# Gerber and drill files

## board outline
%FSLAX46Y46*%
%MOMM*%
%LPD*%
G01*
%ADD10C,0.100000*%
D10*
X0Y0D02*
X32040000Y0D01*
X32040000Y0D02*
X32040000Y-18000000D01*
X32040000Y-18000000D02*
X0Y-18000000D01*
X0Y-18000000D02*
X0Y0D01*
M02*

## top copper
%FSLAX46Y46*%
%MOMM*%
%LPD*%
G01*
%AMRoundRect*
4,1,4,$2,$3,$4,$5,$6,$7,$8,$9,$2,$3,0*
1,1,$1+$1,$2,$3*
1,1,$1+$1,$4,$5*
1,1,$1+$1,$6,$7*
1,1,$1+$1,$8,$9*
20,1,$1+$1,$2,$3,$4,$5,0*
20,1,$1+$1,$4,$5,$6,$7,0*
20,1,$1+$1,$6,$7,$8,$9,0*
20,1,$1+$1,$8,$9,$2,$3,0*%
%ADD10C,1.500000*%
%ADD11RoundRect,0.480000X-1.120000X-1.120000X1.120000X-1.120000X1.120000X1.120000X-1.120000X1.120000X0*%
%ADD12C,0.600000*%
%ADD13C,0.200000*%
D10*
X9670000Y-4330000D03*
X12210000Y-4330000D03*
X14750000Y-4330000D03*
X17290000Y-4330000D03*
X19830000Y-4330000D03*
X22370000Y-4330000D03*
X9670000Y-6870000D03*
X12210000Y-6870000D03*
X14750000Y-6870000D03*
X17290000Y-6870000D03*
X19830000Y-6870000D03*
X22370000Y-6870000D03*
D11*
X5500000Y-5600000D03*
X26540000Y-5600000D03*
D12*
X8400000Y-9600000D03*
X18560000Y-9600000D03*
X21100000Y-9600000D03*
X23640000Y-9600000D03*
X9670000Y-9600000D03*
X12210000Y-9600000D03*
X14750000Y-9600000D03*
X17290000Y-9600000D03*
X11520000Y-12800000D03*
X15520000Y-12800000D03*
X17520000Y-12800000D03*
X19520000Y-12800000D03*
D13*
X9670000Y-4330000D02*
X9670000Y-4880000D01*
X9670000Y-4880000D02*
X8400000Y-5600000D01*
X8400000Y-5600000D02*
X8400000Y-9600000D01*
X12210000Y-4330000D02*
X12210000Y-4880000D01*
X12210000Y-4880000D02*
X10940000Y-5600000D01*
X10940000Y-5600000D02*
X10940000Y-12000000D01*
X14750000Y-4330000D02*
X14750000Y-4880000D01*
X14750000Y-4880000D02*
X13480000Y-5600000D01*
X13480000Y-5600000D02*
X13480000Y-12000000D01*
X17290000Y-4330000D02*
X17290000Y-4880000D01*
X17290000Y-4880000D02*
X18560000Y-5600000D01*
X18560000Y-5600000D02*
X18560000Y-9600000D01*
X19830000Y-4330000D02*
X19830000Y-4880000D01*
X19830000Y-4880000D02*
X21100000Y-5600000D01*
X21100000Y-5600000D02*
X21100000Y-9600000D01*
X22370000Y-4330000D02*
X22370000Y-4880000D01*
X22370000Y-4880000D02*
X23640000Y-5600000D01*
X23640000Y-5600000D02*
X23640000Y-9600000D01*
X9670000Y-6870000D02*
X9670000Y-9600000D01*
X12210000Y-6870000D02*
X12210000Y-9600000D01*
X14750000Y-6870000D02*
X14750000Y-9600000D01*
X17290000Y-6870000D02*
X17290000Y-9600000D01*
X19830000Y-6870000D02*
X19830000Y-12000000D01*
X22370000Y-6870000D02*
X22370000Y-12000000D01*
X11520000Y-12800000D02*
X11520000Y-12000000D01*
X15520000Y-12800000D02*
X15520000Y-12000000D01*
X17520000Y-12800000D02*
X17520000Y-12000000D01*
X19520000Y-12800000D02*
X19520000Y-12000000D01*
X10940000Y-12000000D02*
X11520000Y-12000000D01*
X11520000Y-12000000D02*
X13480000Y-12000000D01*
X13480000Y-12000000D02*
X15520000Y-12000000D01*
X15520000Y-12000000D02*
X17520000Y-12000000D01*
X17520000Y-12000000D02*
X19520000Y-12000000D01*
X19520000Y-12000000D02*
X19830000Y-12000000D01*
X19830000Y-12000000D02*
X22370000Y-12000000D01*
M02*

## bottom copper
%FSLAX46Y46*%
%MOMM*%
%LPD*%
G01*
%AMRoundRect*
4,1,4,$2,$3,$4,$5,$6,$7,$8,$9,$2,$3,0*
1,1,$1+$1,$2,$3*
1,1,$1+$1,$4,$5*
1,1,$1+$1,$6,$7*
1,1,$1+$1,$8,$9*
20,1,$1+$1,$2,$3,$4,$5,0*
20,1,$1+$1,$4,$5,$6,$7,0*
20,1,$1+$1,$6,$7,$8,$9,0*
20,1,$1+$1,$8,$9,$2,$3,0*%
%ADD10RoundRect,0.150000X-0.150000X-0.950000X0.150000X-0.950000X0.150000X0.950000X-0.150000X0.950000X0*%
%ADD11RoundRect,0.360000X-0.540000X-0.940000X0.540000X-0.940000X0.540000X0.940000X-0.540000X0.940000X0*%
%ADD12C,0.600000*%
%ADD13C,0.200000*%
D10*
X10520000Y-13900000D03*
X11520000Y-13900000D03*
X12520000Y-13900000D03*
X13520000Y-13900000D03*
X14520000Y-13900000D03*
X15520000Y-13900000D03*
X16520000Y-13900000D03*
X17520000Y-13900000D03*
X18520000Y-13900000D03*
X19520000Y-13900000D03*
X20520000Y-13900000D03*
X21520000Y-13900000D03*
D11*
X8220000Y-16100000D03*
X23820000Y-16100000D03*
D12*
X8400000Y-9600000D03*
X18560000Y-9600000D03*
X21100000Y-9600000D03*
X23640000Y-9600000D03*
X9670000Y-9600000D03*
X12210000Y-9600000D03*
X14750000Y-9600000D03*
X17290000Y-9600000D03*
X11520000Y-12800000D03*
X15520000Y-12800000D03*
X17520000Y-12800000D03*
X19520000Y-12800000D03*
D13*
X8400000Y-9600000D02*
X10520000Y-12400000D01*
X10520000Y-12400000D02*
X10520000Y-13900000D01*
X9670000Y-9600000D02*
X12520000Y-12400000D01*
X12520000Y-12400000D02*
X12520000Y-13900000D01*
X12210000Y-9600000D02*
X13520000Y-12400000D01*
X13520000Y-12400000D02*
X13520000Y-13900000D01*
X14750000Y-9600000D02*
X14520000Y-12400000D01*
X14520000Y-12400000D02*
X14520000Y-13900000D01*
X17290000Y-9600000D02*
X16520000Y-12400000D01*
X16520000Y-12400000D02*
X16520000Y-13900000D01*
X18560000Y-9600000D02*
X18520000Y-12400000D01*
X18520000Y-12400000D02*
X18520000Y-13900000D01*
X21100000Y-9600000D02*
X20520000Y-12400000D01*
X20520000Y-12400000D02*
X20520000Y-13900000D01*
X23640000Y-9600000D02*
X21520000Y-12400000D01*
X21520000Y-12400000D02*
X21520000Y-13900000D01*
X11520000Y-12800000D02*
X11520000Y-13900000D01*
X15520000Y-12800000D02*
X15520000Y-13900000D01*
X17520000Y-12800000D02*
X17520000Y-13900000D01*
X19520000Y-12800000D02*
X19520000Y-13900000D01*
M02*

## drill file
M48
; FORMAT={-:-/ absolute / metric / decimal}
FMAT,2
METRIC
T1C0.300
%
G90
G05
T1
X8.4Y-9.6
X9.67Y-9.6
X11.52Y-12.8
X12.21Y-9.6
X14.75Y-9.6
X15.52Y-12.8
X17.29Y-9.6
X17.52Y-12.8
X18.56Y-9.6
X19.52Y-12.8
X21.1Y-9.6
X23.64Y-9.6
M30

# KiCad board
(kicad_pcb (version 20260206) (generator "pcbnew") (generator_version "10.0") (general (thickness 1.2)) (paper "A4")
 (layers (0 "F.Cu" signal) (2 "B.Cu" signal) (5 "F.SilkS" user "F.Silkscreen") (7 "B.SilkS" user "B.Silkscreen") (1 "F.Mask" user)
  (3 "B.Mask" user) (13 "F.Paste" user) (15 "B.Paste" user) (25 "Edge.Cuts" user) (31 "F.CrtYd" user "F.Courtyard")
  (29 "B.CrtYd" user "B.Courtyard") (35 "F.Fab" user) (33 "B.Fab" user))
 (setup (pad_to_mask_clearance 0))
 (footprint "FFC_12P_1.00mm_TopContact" (at 16.02 15) (layer "B.Cu")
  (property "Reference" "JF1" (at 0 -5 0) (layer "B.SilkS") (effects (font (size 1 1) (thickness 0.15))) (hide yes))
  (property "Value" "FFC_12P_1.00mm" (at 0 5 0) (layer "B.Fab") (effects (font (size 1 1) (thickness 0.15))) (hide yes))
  (pad "1" smd roundrect (at -5.500 -1.1) (size 0.6 2.2) (layers "B.Cu" "B.Mask" "B.Paste") (roundrect_rratio 0.25) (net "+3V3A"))
  (pad "2" smd roundrect (at -4.500 -1.1) (size 0.6 2.2) (layers "B.Cu" "B.Mask" "B.Paste") (roundrect_rratio 0.25) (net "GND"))
  (pad "3" smd roundrect (at -3.500 -1.1) (size 0.6 2.2) (layers "B.Cu" "B.Mask" "B.Paste") (roundrect_rratio 0.25) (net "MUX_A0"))
  (pad "4" smd roundrect (at -2.500 -1.1) (size 0.6 2.2) (layers "B.Cu" "B.Mask" "B.Paste") (roundrect_rratio 0.25) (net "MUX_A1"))
  (pad "5" smd roundrect (at -1.500 -1.1) (size 0.6 2.2) (layers "B.Cu" "B.Mask" "B.Paste") (roundrect_rratio 0.25) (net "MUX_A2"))
  (pad "6" smd roundrect (at -0.500 -1.1) (size 0.6 2.2) (layers "B.Cu" "B.Mask" "B.Paste") (roundrect_rratio 0.25) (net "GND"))
  (pad "7" smd roundrect (at 0.500 -1.1) (size 0.6 2.2) (layers "B.Cu" "B.Mask" "B.Paste") (roundrect_rratio 0.25) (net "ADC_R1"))
  (pad "8" smd roundrect (at 1.500 -1.1) (size 0.6 2.2) (layers "B.Cu" "B.Mask" "B.Paste") (roundrect_rratio 0.25) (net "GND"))
  (pad "9" smd roundrect (at 2.500 -1.1) (size 0.6 2.2) (layers "B.Cu" "B.Mask" "B.Paste") (roundrect_rratio 0.25) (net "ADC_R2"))
  (pad "10" smd roundrect (at 3.500 -1.1) (size 0.6 2.2) (layers "B.Cu" "B.Mask" "B.Paste") (roundrect_rratio 0.25) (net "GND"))
  (pad "11" smd roundrect (at 4.500 -1.1) (size 0.6 2.2) (layers "B.Cu" "B.Mask" "B.Paste") (roundrect_rratio 0.25) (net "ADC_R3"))
  (pad "12" smd roundrect (at 5.500 -1.1) (size 0.6 2.2) (layers "B.Cu" "B.Mask" "B.Paste") (roundrect_rratio 0.25) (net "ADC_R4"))
  (pad "MP" smd roundrect (at -7.800 1.1) (size 1.8 2.6) (layers "B.Cu" "B.Mask" "B.Paste") (roundrect_rratio 0.2))
  (pad "MP" smd roundrect (at 7.800 1.1) (size 1.8 2.6) (layers "B.Cu" "B.Mask" "B.Paste") (roundrect_rratio 0.2)))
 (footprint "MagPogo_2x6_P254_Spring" (at 16.02 5.6) (layer "F.Cu")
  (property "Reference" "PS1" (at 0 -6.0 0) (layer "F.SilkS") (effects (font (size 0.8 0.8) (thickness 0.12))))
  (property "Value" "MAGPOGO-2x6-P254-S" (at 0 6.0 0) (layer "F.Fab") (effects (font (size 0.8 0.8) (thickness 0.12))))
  (pad "1" smd circle (at -6.35 -1.27) (size 1.5 1.5) (layers "F.Cu" "F.Paste" "F.Mask") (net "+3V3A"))
  (pad "2" smd circle (at -3.81 -1.27) (size 1.5 1.5) (layers "F.Cu" "F.Paste" "F.Mask") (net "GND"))
  (pad "3" smd circle (at -1.27 -1.27) (size 1.5 1.5) (layers "F.Cu" "F.Paste" "F.Mask") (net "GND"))
  (pad "4" smd circle (at 1.27 -1.27) (size 1.5 1.5) (layers "F.Cu" "F.Paste" "F.Mask") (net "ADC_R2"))
  (pad "5" smd circle (at 3.81 -1.27) (size 1.5 1.5) (layers "F.Cu" "F.Paste" "F.Mask") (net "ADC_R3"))
  (pad "6" smd circle (at 6.35 -1.27) (size 1.5 1.5) (layers "F.Cu" "F.Paste" "F.Mask") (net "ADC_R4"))
  (pad "7" smd circle (at -6.35 1.27) (size 1.5 1.5) (layers "F.Cu" "F.Paste" "F.Mask") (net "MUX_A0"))
  (pad "8" smd circle (at -3.81 1.27) (size 1.5 1.5) (layers "F.Cu" "F.Paste" "F.Mask") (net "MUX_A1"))
  (pad "9" smd circle (at -1.27 1.27) (size 1.5 1.5) (layers "F.Cu" "F.Paste" "F.Mask") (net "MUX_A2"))
  (pad "10" smd circle (at 1.27 1.27) (size 1.5 1.5) (layers "F.Cu" "F.Paste" "F.Mask") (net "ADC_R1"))
  (pad "11" smd circle (at 3.81 1.27) (size 1.5 1.5) (layers "F.Cu" "F.Paste" "F.Mask") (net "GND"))
  (pad "12" smd circle (at 6.35 1.27) (size 1.5 1.5) (layers "F.Cu" "F.Paste" "F.Mask") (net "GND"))
  (pad "MP1" smd roundrect (at -10.52 0) (size 3.2 3.2) (roundrect_rratio 0.15) (layers "F.Cu" "F.Paste" "F.Mask"))
  (pad "MP2" smd roundrect (at 10.52 0) (size 3.2 3.2) (roundrect_rratio 0.15) (layers "F.Cu" "F.Paste" "F.Mask")))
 (gr_line (start 0 0) (end 32.04 0) (stroke (width 0.1) (type solid)) (layer "Edge.Cuts"))
 (gr_line (start 32.04 0) (end 32.04 18) (stroke (width 0.1) (type solid)) (layer "Edge.Cuts"))
 (gr_line (start 32.04 18) (end 0 18) (stroke (width 0.1) (type solid)) (layer "Edge.Cuts"))
 (gr_line (start 0 18) (end 0 0) (stroke (width 0.1) (type solid)) (layer "Edge.Cuts"))
 (segment (start 9.67 4.33) (end 9.67 4.88) (width 0.2) (layer "F.Cu") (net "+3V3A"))
 (segment (start 9.67 4.88) (end 8.4 5.6) (width 0.2) (layer "F.Cu") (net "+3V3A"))
 (segment (start 8.4 5.6) (end 8.4 9.6) (width 0.2) (layer "F.Cu") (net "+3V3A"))
 (via (at 8.4 9.6) (size 0.6) (drill 0.3) (layers "F.Cu" "B.Cu") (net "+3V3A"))
 (segment (start 12.21 4.33) (end 12.21 4.88) (width 0.2) (layer "F.Cu") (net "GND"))
 (segment (start 12.21 4.88) (end 10.94 5.6) (width 0.2) (layer "F.Cu") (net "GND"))
 (segment (start 10.94 5.6) (end 10.94 12) (width 0.2) (layer "F.Cu") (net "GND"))
 (segment (start 14.75 4.33) (end 14.75 4.88) (width 0.2) (layer "F.Cu") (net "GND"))
 (segment (start 14.75 4.88) (end 13.48 5.6) (width 0.2) (layer "F.Cu") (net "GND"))
 (segment (start 13.48 5.6) (end 13.48 12) (width 0.2) (layer "F.Cu") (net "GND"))
 (segment (start 17.29 4.33) (end 17.29 4.88) (width 0.2) (layer "F.Cu") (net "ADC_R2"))
 (segment (start 17.29 4.88) (end 18.56 5.6) (width 0.2) (layer "F.Cu") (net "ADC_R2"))
 (segment (start 18.56 5.6) (end 18.56 9.6) (width 0.2) (layer "F.Cu") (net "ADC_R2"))
 (via (at 18.56 9.6) (size 0.6) (drill 0.3) (layers "F.Cu" "B.Cu") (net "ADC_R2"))
 (segment (start 19.83 4.33) (end 19.83 4.88) (width 0.2) (layer "F.Cu") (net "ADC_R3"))
 (segment (start 19.83 4.88) (end 21.1 5.6) (width 0.2) (layer "F.Cu") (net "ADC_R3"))
 (segment (start 21.1 5.6) (end 21.1 9.6) (width 0.2) (layer "F.Cu") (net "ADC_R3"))
 (via (at 21.1 9.6) (size 0.6) (drill 0.3) (layers "F.Cu" "B.Cu") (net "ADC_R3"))
 (segment (start 22.37 4.33) (end 22.37 4.88) (width 0.2) (layer "F.Cu") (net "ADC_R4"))
 (segment (start 22.37 4.88) (end 23.64 5.6) (width 0.2) (layer "F.Cu") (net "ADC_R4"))
 (segment (start 23.64 5.6) (end 23.64 9.6) (width 0.2) (layer "F.Cu") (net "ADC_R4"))
 (via (at 23.64 9.6) (size 0.6) (drill 0.3) (layers "F.Cu" "B.Cu") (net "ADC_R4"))
 (segment (start 9.67 6.87) (end 9.67 9.6) (width 0.2) (layer "F.Cu") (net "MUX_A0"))
 (via (at 9.67 9.6) (size 0.6) (drill 0.3) (layers "F.Cu" "B.Cu") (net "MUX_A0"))
 (segment (start 12.21 6.87) (end 12.21 9.6) (width 0.2) (layer "F.Cu") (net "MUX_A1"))
 (via (at 12.21 9.6) (size 0.6) (drill 0.3) (layers "F.Cu" "B.Cu") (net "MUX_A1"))
 (segment (start 14.75 6.87) (end 14.75 9.6) (width 0.2) (layer "F.Cu") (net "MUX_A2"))
 (via (at 14.75 9.6) (size 0.6) (drill 0.3) (layers "F.Cu" "B.Cu") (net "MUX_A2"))
 (segment (start 17.29 6.87) (end 17.29 9.6) (width 0.2) (layer "F.Cu") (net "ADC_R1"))
 (via (at 17.29 9.6) (size 0.6) (drill 0.3) (layers "F.Cu" "B.Cu") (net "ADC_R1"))
 (segment (start 19.83 6.87) (end 19.83 12) (width 0.2) (layer "F.Cu") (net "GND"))
 (segment (start 22.37 6.87) (end 22.37 12) (width 0.2) (layer "F.Cu") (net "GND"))
 (segment (start 8.4 9.6) (end 10.52 12.4) (width 0.2) (layer "B.Cu") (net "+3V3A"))
 (segment (start 10.52 12.4) (end 10.52 13.9) (width 0.2) (layer "B.Cu") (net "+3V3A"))
 (segment (start 9.67 9.6) (end 12.52 12.4) (width 0.2) (layer "B.Cu") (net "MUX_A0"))
 (segment (start 12.52 12.4) (end 12.52 13.9) (width 0.2) (layer "B.Cu") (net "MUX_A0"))
 (segment (start 12.21 9.6) (end 13.52 12.4) (width 0.2) (layer "B.Cu") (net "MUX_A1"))
 (segment (start 13.52 12.4) (end 13.52 13.9) (width 0.2) (layer "B.Cu") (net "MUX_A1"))
 (segment (start 14.75 9.6) (end 14.52 12.4) (width 0.2) (layer "B.Cu") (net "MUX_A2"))
 (segment (start 14.52 12.4) (end 14.52 13.9) (width 0.2) (layer "B.Cu") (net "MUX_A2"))
 (segment (start 17.29 9.6) (end 16.52 12.4) (width 0.2) (layer "B.Cu") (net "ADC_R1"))
 (segment (start 16.52 12.4) (end 16.52 13.9) (width 0.2) (layer "B.Cu") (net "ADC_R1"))
 (segment (start 18.56 9.6) (end 18.52 12.4) (width 0.2) (layer "B.Cu") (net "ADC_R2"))
 (segment (start 18.52 12.4) (end 18.52 13.9) (width 0.2) (layer "B.Cu") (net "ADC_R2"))
 (segment (start 21.1 9.6) (end 20.52 12.4) (width 0.2) (layer "B.Cu") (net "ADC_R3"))
 (segment (start 20.52 12.4) (end 20.52 13.9) (width 0.2) (layer "B.Cu") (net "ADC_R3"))
 (segment (start 23.64 9.6) (end 21.52 12.4) (width 0.2) (layer "B.Cu") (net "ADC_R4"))
 (segment (start 21.52 12.4) (end 21.52 13.9) (width 0.2) (layer "B.Cu") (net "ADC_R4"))
 (segment (start 11.52 12.8) (end 11.52 13.9) (width 0.2) (layer "B.Cu") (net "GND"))
 (via (at 11.52 12.8) (size 0.6) (drill 0.3) (layers "F.Cu" "B.Cu") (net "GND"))
 (segment (start 11.52 12.8) (end 11.52 12) (width 0.2) (layer "F.Cu") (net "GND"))
 (segment (start 15.52 12.8) (end 15.52 13.9) (width 0.2) (layer "B.Cu") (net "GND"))
 (via (at 15.52 12.8) (size 0.6) (drill 0.3) (layers "F.Cu" "B.Cu") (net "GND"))
 (segment (start 15.52 12.8) (end 15.52 12) (width 0.2) (layer "F.Cu") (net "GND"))
 (segment (start 17.52 12.8) (end 17.52 13.9) (width 0.2) (layer "B.Cu") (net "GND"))
 (via (at 17.52 12.8) (size 0.6) (drill 0.3) (layers "F.Cu" "B.Cu") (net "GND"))
 (segment (start 17.52 12.8) (end 17.52 12) (width 0.2) (layer "F.Cu") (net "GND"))
 (segment (start 19.52 12.8) (end 19.52 13.9) (width 0.2) (layer "B.Cu") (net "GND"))
 (via (at 19.52 12.8) (size 0.6) (drill 0.3) (layers "F.Cu" "B.Cu") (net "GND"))
 (segment (start 19.52 12.8) (end 19.52 12) (width 0.2) (layer "F.Cu") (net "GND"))
 (segment (start 10.94 12) (end 11.52 12) (width 0.2) (layer "F.Cu") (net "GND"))
 (segment (start 11.52 12) (end 13.48 12) (width 0.2) (layer "F.Cu") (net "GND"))
 (segment (start 13.48 12) (end 15.52 12) (width 0.2) (layer "F.Cu") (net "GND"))
 (segment (start 15.52 12) (end 17.52 12) (width 0.2) (layer "F.Cu") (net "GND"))
 (segment (start 17.52 12) (end 19.52 12) (width 0.2) (layer "F.Cu") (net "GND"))
 (segment (start 19.52 12) (end 19.83 12) (width 0.2) (layer "F.Cu") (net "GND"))
 (segment (start 19.83 12) (end 22.37 12) (width 0.2) (layer "F.Cu") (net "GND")))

